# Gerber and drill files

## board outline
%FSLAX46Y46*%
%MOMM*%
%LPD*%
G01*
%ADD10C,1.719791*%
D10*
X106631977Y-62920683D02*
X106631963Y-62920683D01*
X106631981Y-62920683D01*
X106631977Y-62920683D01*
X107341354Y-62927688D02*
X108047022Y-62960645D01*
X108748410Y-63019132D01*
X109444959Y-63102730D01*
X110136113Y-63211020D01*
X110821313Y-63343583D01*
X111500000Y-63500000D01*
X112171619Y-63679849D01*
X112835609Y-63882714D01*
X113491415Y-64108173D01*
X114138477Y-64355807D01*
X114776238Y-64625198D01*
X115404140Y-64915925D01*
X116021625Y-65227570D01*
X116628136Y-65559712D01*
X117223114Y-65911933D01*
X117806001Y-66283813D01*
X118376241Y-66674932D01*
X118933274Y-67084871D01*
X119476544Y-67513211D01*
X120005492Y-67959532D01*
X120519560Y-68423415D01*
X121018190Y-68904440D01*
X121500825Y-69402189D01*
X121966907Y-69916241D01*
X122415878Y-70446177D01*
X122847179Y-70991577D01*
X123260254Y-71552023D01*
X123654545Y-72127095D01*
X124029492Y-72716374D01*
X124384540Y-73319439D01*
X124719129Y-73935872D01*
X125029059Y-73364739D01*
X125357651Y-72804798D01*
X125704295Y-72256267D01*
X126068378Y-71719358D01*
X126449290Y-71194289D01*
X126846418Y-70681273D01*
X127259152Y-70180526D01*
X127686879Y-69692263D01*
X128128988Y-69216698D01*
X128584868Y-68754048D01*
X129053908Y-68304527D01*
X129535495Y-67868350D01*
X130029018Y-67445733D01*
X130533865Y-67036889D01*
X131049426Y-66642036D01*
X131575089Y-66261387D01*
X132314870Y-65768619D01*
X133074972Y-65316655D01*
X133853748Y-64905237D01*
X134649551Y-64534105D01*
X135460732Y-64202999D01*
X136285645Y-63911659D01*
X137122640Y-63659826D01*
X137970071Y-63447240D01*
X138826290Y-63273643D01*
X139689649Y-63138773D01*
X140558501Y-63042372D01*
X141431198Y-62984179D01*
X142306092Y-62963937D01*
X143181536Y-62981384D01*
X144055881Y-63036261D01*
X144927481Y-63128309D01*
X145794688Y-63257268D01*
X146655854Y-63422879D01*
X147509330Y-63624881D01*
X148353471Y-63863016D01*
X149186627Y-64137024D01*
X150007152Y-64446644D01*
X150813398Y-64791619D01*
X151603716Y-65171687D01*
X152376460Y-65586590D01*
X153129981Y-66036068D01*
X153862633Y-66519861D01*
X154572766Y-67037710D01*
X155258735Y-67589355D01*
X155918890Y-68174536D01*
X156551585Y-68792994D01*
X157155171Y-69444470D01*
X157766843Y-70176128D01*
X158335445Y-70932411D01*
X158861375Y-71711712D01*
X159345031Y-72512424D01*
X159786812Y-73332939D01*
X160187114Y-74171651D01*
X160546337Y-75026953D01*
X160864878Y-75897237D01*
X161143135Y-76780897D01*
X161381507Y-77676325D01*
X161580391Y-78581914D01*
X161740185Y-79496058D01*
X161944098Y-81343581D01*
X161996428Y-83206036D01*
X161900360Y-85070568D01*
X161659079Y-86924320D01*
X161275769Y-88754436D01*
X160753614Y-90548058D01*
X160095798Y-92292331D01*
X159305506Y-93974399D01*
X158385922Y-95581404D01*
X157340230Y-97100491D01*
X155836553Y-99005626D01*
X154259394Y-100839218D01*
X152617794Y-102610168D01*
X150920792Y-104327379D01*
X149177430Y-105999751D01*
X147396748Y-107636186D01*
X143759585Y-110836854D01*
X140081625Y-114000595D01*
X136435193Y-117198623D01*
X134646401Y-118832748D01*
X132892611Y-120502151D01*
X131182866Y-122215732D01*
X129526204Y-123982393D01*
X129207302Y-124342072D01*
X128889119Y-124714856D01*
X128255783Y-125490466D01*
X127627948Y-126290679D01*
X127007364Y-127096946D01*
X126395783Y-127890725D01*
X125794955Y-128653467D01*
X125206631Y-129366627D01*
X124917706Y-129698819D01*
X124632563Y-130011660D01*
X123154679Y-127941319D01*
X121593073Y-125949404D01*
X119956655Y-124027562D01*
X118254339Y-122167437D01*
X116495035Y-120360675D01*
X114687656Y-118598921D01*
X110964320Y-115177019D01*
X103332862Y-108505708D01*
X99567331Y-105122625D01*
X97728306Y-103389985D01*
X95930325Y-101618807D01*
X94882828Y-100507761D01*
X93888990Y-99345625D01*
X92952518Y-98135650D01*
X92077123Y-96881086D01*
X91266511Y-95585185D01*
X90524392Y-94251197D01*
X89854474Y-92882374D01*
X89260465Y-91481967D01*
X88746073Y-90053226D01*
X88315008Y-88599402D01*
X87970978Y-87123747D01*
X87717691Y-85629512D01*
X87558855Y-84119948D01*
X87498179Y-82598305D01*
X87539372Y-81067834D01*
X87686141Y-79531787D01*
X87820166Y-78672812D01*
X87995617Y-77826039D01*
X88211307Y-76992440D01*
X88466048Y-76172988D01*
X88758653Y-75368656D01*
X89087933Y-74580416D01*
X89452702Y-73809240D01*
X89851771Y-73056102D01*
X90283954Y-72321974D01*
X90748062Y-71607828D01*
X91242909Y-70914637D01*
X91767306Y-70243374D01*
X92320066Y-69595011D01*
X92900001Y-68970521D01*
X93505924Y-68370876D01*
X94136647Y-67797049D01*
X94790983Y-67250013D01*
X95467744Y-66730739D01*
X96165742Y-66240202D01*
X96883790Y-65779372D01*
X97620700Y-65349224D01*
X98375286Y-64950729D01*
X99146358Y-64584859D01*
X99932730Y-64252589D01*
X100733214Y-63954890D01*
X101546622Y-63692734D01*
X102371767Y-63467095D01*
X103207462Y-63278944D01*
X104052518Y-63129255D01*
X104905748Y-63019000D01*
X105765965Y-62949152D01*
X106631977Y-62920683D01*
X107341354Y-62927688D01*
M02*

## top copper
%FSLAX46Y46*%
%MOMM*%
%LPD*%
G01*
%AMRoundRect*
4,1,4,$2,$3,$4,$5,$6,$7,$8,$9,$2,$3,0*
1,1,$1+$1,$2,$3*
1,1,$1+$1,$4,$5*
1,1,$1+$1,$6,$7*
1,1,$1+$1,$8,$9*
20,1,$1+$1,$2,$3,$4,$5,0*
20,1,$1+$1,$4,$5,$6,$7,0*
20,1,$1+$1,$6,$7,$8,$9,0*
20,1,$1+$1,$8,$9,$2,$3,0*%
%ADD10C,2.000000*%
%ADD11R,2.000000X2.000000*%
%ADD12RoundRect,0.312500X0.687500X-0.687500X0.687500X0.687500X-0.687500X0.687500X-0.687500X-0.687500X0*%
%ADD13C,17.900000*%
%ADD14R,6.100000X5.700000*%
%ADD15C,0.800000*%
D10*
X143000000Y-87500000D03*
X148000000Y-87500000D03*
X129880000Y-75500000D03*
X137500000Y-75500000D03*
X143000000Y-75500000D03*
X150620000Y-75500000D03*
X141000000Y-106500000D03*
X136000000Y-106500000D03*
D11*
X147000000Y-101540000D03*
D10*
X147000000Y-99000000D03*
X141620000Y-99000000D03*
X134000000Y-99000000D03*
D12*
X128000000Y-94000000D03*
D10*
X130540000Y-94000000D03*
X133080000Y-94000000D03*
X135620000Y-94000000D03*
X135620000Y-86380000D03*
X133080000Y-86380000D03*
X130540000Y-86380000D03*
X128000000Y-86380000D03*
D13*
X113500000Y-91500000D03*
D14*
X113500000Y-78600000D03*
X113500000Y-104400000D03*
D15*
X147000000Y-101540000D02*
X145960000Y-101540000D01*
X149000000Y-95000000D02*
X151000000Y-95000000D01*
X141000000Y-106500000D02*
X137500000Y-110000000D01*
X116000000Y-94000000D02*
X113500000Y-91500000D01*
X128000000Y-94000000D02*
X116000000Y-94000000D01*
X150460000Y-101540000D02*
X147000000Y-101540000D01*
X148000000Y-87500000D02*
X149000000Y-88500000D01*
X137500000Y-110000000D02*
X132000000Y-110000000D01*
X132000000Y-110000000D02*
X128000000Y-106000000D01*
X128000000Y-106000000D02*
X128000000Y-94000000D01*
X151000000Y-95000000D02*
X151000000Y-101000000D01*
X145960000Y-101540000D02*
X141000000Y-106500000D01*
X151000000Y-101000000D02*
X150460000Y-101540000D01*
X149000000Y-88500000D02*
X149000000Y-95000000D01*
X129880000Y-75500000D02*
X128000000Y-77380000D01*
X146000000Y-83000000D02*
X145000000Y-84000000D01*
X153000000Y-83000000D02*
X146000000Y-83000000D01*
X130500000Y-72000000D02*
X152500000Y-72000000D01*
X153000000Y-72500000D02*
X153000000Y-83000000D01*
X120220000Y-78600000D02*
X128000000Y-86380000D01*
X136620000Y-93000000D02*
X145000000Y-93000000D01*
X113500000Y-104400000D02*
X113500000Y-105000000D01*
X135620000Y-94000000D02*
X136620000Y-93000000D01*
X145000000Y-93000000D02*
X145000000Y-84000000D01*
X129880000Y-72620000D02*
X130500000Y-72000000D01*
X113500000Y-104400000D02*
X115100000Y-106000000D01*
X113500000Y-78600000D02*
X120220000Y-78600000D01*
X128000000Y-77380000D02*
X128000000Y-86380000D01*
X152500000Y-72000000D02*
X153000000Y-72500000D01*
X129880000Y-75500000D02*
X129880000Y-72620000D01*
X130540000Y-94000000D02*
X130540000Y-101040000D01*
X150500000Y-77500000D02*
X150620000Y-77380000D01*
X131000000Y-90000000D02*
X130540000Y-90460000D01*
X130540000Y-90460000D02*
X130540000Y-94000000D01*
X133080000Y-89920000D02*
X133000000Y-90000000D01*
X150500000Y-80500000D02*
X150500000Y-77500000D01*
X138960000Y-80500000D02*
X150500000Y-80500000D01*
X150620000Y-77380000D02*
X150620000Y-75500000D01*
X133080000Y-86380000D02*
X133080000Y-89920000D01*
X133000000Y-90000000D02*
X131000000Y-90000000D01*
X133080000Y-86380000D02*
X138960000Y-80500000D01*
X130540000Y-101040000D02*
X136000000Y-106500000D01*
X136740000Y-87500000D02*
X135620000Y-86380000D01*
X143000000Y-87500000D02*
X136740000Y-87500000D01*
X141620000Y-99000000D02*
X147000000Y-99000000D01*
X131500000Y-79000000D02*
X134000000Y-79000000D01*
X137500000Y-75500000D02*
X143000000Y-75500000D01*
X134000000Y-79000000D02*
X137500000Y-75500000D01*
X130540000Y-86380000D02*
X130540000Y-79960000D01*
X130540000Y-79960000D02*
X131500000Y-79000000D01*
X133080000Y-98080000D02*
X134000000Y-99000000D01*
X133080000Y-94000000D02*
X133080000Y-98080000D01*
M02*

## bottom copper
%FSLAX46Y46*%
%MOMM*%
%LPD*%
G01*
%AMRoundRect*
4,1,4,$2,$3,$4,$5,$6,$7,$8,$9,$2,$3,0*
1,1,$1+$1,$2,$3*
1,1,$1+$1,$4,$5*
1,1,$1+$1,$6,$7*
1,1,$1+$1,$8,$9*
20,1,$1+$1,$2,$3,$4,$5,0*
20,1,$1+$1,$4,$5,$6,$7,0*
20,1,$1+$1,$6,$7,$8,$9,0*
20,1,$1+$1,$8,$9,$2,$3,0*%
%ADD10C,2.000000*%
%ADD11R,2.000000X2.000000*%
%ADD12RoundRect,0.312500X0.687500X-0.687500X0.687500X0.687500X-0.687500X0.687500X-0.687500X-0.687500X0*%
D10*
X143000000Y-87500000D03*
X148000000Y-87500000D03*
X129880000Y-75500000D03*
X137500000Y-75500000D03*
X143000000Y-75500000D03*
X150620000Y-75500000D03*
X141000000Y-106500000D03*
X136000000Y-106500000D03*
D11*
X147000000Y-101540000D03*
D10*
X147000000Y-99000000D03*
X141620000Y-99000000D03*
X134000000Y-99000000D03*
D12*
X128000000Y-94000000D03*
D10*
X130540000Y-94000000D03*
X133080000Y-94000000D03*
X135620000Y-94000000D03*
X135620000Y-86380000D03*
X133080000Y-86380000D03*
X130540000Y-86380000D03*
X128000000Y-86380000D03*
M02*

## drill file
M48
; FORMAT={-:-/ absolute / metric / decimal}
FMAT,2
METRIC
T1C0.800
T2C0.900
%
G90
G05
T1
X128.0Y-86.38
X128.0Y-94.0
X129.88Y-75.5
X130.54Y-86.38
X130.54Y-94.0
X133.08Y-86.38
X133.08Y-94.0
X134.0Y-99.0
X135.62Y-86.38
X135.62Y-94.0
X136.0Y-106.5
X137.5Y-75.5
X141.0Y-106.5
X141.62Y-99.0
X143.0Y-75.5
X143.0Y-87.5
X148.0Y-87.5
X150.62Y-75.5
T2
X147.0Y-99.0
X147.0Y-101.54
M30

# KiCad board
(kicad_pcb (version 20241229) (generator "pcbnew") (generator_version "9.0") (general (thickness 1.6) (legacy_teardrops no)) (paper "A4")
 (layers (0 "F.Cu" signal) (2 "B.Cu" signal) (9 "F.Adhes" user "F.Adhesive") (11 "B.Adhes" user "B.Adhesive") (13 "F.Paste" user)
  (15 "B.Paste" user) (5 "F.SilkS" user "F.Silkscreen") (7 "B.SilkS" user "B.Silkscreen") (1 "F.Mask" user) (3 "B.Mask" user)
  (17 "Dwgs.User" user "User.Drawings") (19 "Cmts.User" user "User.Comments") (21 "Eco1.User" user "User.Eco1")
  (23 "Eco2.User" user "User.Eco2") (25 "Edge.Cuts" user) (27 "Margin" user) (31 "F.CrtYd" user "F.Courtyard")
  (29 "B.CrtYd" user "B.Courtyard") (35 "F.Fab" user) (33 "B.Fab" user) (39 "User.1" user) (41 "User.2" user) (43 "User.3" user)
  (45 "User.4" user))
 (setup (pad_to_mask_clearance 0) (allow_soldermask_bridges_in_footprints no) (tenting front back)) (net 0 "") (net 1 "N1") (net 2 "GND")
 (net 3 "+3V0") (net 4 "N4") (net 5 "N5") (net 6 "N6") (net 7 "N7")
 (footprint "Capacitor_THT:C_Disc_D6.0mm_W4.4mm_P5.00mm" (layer "F.Cu") (at 143 87.5)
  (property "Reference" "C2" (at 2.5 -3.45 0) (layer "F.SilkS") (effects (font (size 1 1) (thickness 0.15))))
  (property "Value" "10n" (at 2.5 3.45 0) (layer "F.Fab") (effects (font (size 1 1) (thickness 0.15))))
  (pad "1" thru_hole circle (at 0 0) (size 2 2) (drill 0.8) (layers "*.Cu" "*.Mask") (remove_unused_layers no) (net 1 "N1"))
  (pad "2" thru_hole circle (at 5 0) (size 2 2) (drill 0.8) (layers "*.Cu" "*.Mask") (remove_unused_layers no) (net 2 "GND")))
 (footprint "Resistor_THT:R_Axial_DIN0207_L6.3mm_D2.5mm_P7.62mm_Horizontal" (layer "F.Cu") (at 129.88 75.5)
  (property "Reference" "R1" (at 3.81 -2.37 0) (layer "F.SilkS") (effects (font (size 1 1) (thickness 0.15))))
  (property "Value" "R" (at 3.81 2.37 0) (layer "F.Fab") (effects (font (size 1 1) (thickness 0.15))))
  (pad "1" thru_hole circle (at 0 0) (size 2 2) (drill 0.8) (layers "*.Cu" "*.Mask") (remove_unused_layers no) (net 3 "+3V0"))
  (pad "2" thru_hole circle (at 7.62 0) (size 2 2) (drill 0.8) (layers "*.Cu" "*.Mask") (remove_unused_layers no) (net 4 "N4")))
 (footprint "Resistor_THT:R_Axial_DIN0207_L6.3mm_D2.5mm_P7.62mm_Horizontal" (layer "F.Cu") (at 143 75.5)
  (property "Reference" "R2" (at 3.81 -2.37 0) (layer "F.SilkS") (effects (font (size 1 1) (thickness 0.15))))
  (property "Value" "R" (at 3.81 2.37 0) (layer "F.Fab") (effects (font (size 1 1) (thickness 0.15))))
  (pad "1" thru_hole circle (at 0 0) (size 2 2) (drill 0.8) (layers "*.Cu" "*.Mask") (remove_unused_layers no) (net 4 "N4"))
  (pad "2" thru_hole circle (at 7.62 0) (size 2 2) (drill 0.8) (layers "*.Cu" "*.Mask") (remove_unused_layers no) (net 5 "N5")))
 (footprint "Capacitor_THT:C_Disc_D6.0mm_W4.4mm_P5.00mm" (layer "F.Cu") (at 141 106.5 180)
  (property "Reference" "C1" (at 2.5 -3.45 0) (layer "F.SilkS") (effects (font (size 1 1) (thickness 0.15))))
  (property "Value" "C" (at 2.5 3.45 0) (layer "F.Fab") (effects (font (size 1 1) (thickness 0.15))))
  (pad "1" thru_hole circle (at 0 0 180) (size 2 2) (drill 0.8) (layers "*.Cu" "*.Mask") (remove_unused_layers no) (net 2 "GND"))
  (pad "2" thru_hole circle (at 5 0 180) (size 2 2) (drill 0.8) (layers "*.Cu" "*.Mask") (remove_unused_layers no) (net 5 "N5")))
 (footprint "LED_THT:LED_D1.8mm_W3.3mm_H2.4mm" (layer "F.Cu") (at 147 101.54 90)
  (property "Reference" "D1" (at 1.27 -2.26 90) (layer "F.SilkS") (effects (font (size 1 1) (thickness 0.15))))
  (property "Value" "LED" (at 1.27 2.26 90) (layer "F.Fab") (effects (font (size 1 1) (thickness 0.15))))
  (pad "1" thru_hole rect (at 0 0 90) (size 2 2) (drill 0.9) (layers "*.Cu" "*.Mask") (remove_unused_layers no) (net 2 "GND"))
  (pad "2" thru_hole circle (at 2.54 0 90) (size 2 2) (drill 0.9) (layers "*.Cu" "*.Mask") (remove_unused_layers no) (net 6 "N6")))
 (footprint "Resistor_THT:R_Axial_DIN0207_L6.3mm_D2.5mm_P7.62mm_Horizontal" (layer "F.Cu") (at 141.62 99 180)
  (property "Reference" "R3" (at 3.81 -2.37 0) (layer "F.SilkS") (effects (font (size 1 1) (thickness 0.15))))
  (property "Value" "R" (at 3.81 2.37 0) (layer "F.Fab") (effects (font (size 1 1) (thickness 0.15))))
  (pad "1" thru_hole circle (at 0 0 180) (size 2 2) (drill 0.8) (layers "*.Cu" "*.Mask") (remove_unused_layers no) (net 6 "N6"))
  (pad "2" thru_hole circle (at 7.62 0 180) (size 2 2) (drill 0.8) (layers "*.Cu" "*.Mask") (remove_unused_layers no) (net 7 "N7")))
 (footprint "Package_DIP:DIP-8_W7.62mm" (layer "F.Cu") (at 128 94 90)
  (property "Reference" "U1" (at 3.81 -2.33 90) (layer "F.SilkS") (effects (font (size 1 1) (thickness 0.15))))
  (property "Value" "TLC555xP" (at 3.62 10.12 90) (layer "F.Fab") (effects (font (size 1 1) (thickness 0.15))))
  (pad "1" thru_hole roundrect (at 0 0 90) (size 2 2) (drill 0.8) (layers "*.Cu" "*.Mask") (remove_unused_layers no)
   (roundrect_rratio 0.15625) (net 2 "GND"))
  (pad "2" thru_hole circle (at 0 2.54 90) (size 2 2) (drill 0.8) (layers "*.Cu" "*.Mask") (remove_unused_layers no) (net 5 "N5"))
  (pad "3" thru_hole circle (at 0 5.08 90) (size 2 2) (drill 0.8) (layers "*.Cu" "*.Mask") (remove_unused_layers no) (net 7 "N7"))
  (pad "4" thru_hole circle (at 0 7.62 90) (size 2 2) (drill 0.8) (layers "*.Cu" "*.Mask") (remove_unused_layers no) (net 3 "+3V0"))
  (pad "5" thru_hole circle (at 7.62 7.62 90) (size 2 2) (drill 0.8) (layers "*.Cu" "*.Mask") (remove_unused_layers no) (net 1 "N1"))
  (pad "6" thru_hole circle (at 7.62 5.08 90) (size 2 2) (drill 0.8) (layers "*.Cu" "*.Mask") (remove_unused_layers no) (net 5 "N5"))
  (pad "7" thru_hole circle (at 7.62 2.54 90) (size 2 2) (drill 0.8) (layers "*.Cu" "*.Mask") (remove_unused_layers no) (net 4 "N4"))
  (pad "8" thru_hole circle (at 7.62 0 90) (size 2 2) (drill 0.8) (layers "*.Cu" "*.Mask") (remove_unused_layers no) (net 3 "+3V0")))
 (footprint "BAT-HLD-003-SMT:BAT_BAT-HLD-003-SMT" (layer "F.Cu") (at 113.5 91.5 -90)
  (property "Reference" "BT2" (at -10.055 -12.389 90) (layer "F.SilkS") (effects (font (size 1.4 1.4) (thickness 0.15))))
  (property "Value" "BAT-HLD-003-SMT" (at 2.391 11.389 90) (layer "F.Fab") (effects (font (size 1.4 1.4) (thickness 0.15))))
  (pad "N" smd circle (at 0 0 270) (size 17.9 17.9) (layers "F.Cu" "F.Mask") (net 2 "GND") (solder_mask_margin 0.102))
  (pad "P1" smd rect (at -12.9 0 270) (size 5.7 6.1) (layers "F.Cu" "F.Mask" "F.Paste") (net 3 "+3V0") (solder_mask_margin 0.102))
  (pad "P2" smd rect (at 12.9 0 270) (size 5.7 6.1) (layers "F.Cu" "F.Mask" "F.Paste") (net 3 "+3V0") (solder_mask_margin 0.102)))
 (gr_poly
  (pts (xy 106.631977 62.920683) (xy 106.631963 62.920683) (xy 106.631981 62.920683)) (stroke (width 1.719791) (type solid)) (fill no)
  (layer "Edge.Cuts"))
 (gr_poly
  (pts (xy 107.341354 62.927688) (xy 108.047022 62.960645) (xy 108.74841 63.019132) (xy 109.444959 63.10273) (xy 110.136113 63.21102)
   (xy 110.821313 63.343583) (xy 111.5 63.5) (xy 112.171619 63.679849) (xy 112.835609 63.882714) (xy 113.491415 64.108173)
   (xy 114.138477 64.355807) (xy 114.776238 64.625198) (xy 115.40414 64.915925) (xy 116.021625 65.22757) (xy 116.628136 65.559712)
   (xy 117.223114 65.911933) (xy 117.806001 66.283813) (xy 118.376241 66.674932) (xy 118.933274 67.084871) (xy 119.476544 67.513211)
   (xy 120.005492 67.959532) (xy 120.51956 68.423415) (xy 121.01819 68.90444) (xy 121.500825 69.402189) (xy 121.966907 69.916241)
   (xy 122.415878 70.446177) (xy 122.847179 70.991577) (xy 123.260254 71.552023) (xy 123.654545 72.127095) (xy 124.029492 72.716374)
   (xy 124.38454 73.319439) (xy 124.719129 73.935872) (xy 125.029059 73.364739) (xy 125.357651 72.804798) (xy 125.704295 72.256267)
   (xy 126.068378 71.719358) (xy 126.44929 71.194289) (xy 126.846418 70.681273) (xy 127.259152 70.180526) (xy 127.686879 69.692263)
   (xy 128.128988 69.216698) (xy 128.584868 68.754048) (xy 129.053908 68.304527) (xy 129.535495 67.86835) (xy 130.029018 67.445733)
   (xy 130.533865 67.036889) (xy 131.049426 66.642036) (xy 131.575089 66.261387) (xy 132.31487 65.768619) (xy 133.074972 65.316655)
   (xy 133.853748 64.905237) (xy 134.649551 64.534105) (xy 135.460732 64.202999) (xy 136.285645 63.911659) (xy 137.12264 63.659826)
   (xy 137.970071 63.44724) (xy 138.82629 63.273643) (xy 139.689649 63.138773) (xy 140.558501 63.042372) (xy 141.431198 62.984179)
   (xy 142.306092 62.963937) (xy 143.181536 62.981384) (xy 144.055881 63.036261) (xy 144.927481 63.128309) (xy 145.794688 63.257268)
   (xy 146.655854 63.422879) (xy 147.50933 63.624881) (xy 148.353471 63.863016) (xy 149.186627 64.137024) (xy 150.007152 64.446644)
   (xy 150.813398 64.791619) (xy 151.603716 65.171687) (xy 152.37646 65.58659) (xy 153.129981 66.036068) (xy 153.862633 66.519861)
   (xy 154.572766 67.03771) (xy 155.258735 67.589355) (xy 155.91889 68.174536) (xy 156.551585 68.792994) (xy 157.155171 69.44447)
   (xy 157.766843 70.176128) (xy 158.335445 70.932411) (xy 158.861375 71.711712) (xy 159.345031 72.512424) (xy 159.786812 73.332939)
   (xy 160.187114 74.171651) (xy 160.546337 75.026953) (xy 160.864878 75.897237) (xy 161.143135 76.780897) (xy 161.381507 77.676325)
   (xy 161.580391 78.581914) (xy 161.740185 79.496058) (xy 161.944098 81.343581) (xy 161.996428 83.206036) (xy 161.90036 85.070568)
   (xy 161.659079 86.92432) (xy 161.275769 88.754436) (xy 160.753614 90.548058) (xy 160.095798 92.292331) (xy 159.305506 93.974399)
   (xy 158.385922 95.581404) (xy 157.34023 97.100491) (xy 155.836553 99.005626) (xy 154.259394 100.839218) (xy 152.617794 102.610168)
   (xy 150.920792 104.327379) (xy 149.17743 105.999751) (xy 147.396748 107.636186) (xy 143.759585 110.836854) (xy 140.081625 114.000595)
   (xy 136.435193 117.198623) (xy 134.646401 118.832748) (xy 132.892611 120.502151) (xy 131.182866 122.215732) (xy 129.526204 123.982393)
   (xy 129.207302 124.342072) (xy 128.889119 124.714856) (xy 128.255783 125.490466) (xy 127.627948 126.290679) (xy 127.007364 127.096946)
   (xy 126.395783 127.890725) (xy 125.794955 128.653467) (xy 125.206631 129.366627) (xy 124.917706 129.698819) (xy 124.632563 130.01166)
   (xy 123.154679 127.941319) (xy 121.593073 125.949404) (xy 119.956655 124.027562) (xy 118.254339 122.167437) (xy 116.495035 120.360675)
   (xy 114.687656 118.598921) (xy 110.96432 115.177019) (xy 103.332862 108.505708) (xy 99.567331 105.122625) (xy 97.728306 103.389985)
   (xy 95.930325 101.618807) (xy 94.882828 100.507761) (xy 93.88899 99.345625) (xy 92.952518 98.13565) (xy 92.077123 96.881086)
   (xy 91.266511 95.585185) (xy 90.524392 94.251197) (xy 89.854474 92.882374) (xy 89.260465 91.481967) (xy 88.746073 90.053226)
   (xy 88.315008 88.599402) (xy 87.970978 87.123747) (xy 87.717691 85.629512) (xy 87.558855 84.119948) (xy 87.498179 82.598305)
   (xy 87.539372 81.067834) (xy 87.686141 79.531787) (xy 87.820166 78.672812) (xy 87.995617 77.826039) (xy 88.211307 76.99244)
   (xy 88.466048 76.172988) (xy 88.758653 75.368656) (xy 89.087933 74.580416) (xy 89.452702 73.80924) (xy 89.851771 73.056102)
   (xy 90.283954 72.321974) (xy 90.748062 71.607828) (xy 91.242909 70.914637) (xy 91.767306 70.243374) (xy 92.320066 69.595011)
   (xy 92.900001 68.970521) (xy 93.505924 68.370876) (xy 94.136647 67.797049) (xy 94.790983 67.250013) (xy 95.467744 66.730739)
   (xy 96.165742 66.240202) (xy 96.88379 65.779372) (xy 97.6207 65.349224) (xy 98.375286 64.950729) (xy 99.146358 64.584859)
   (xy 99.93273 64.252589) (xy 100.733214 63.95489) (xy 101.546622 63.692734) (xy 102.371767 63.467095) (xy 103.207462 63.278944)
   (xy 104.052518 63.129255) (xy 104.905748 63.019) (xy 105.765965 62.949152) (xy 106.631977 62.920683))
  (stroke (width 1.719791) (type solid)) (fill no) (layer "Edge.Cuts"))
 (segment (start 147 101.54) (end 145.96 101.54) (width 0.8) (layer "F.Cu") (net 2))
 (segment (start 149 95) (end 151 95) (width 0.8) (layer "F.Cu") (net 2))
 (segment (start 141 106.5) (end 137.5 110) (width 0.8) (layer "F.Cu") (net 2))
 (segment (start 116 94) (end 113.5 91.5) (width 0.8) (layer "F.Cu") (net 2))
 (segment (start 128 94) (end 116 94) (width 0.8) (layer "F.Cu") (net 2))
 (segment (start 150.46 101.54) (end 147 101.54) (width 0.8) (layer "F.Cu") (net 2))
 (segment (start 148 87.5) (end 149 88.5) (width 0.8) (layer "F.Cu") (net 2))
 (segment (start 137.5 110) (end 132 110) (width 0.8) (layer "F.Cu") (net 2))
 (segment (start 132 110) (end 128 106) (width 0.8) (layer "F.Cu") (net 2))
 (segment (start 128 106) (end 128 94) (width 0.8) (layer "F.Cu") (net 2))
 (segment (start 151 95) (end 151 101) (width 0.8) (layer "F.Cu") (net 2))
 (segment (start 145.96 101.54) (end 141 106.5) (width 0.8) (layer "F.Cu") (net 2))
 (segment (start 151 101) (end 150.46 101.54) (width 0.8) (layer "F.Cu") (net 2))
 (segment (start 149 88.5) (end 149 95) (width 0.8) (layer "F.Cu") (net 2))
 (segment (start 129.88 75.5) (end 128 77.38) (width 0.8) (layer "F.Cu") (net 3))
 (segment (start 146 83) (end 145 84) (width 0.8) (layer "F.Cu") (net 3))
 (segment (start 153 83) (end 146 83) (width 0.8) (layer "F.Cu") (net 3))
 (segment (start 130.5 72) (end 152.5 72) (width 0.8) (layer "F.Cu") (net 3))
 (segment (start 153 72.5) (end 153 83) (width 0.8) (layer "F.Cu") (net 3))
 (segment (start 120.22 78.6) (end 128 86.38) (width 0.8) (layer "F.Cu") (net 3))
 (segment (start 136.62 93) (end 145 93) (width 0.8) (layer "F.Cu") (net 3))
 (segment (start 113.5 104.4) (end 113.5 105) (width 0.8) (layer "F.Cu") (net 3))
 (segment (start 135.62 94) (end 136.62 93) (width 0.8) (layer "F.Cu") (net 3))
 (segment (start 145 93) (end 145 84) (width 0.8) (layer "F.Cu") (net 3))
 (segment (start 129.88 72.62) (end 130.5 72) (width 0.8) (layer "F.Cu") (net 3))
 (segment (start 113.5 104.4) (end 115.1 106) (width 0.8) (layer "F.Cu") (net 3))
 (segment (start 113.5 78.6) (end 120.22 78.6) (width 0.8) (layer "F.Cu") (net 3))
 (segment (start 128 77.38) (end 128 86.38) (width 0.8) (layer "F.Cu") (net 3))
 (segment (start 152.5 72) (end 153 72.5) (width 0.8) (layer "F.Cu") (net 3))
 (segment (start 129.88 75.5) (end 129.88 72.62) (width 0.8) (layer "F.Cu") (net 3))
 (segment (start 130.54 94) (end 130.54 101.04) (width 0.8) (layer "F.Cu") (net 5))
 (segment (start 150.5 77.5) (end 150.62 77.38) (width 0.8) (layer "F.Cu") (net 5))
 (segment (start 131 90) (end 130.54 90.46) (width 0.8) (layer "F.Cu") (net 5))
 (segment (start 130.54 90.46) (end 130.54 94) (width 0.8) (layer "F.Cu") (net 5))
 (segment (start 133.08 89.92) (end 133 90) (width 0.8) (layer "F.Cu") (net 5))
 (segment (start 150.5 80.5) (end 150.5 77.5) (width 0.8) (layer "F.Cu") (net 5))
 (segment (start 138.96 80.5) (end 150.5 80.5) (width 0.8) (layer "F.Cu") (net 5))
 (segment (start 150.62 77.38) (end 150.62 75.5) (width 0.8) (layer "F.Cu") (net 5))
 (segment (start 133.08 86.38) (end 133.08 89.92) (width 0.8) (layer "F.Cu") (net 5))
 (segment (start 133 90) (end 131 90) (width 0.8) (layer "F.Cu") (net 5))
 (segment (start 133.08 86.38) (end 138.96 80.5) (width 0.8) (layer "F.Cu") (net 5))
 (segment (start 130.54 101.04) (end 136 106.5) (width 0.8) (layer "F.Cu") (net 5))
 (segment (start 136.74 87.5) (end 135.62 86.38) (width 0.8) (layer "F.Cu") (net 1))
 (segment (start 143 87.5) (end 136.74 87.5) (width 0.8) (layer "F.Cu") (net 1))
 (segment (start 141.62 99) (end 147 99) (width 0.8) (layer "F.Cu") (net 6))
 (segment (start 131.5 79) (end 134 79) (width 0.8) (layer "F.Cu") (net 4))
 (segment (start 137.5 75.5) (end 143 75.5) (width 0.8) (layer "F.Cu") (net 4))
 (segment (start 134 79) (end 137.5 75.5) (width 0.8) (layer "F.Cu") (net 4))
 (segment (start 130.54 86.38) (end 130.54 79.96) (width 0.8) (layer "F.Cu") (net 4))
 (segment (start 130.54 79.96) (end 131.5 79) (width 0.8) (layer "F.Cu") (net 4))
 (segment (start 133.08 98.08) (end 134 99) (width 0.8) (layer "F.Cu") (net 7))
 (segment (start 133.08 94) (end 133.08 98.08) (width 0.8) (layer "F.Cu") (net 7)))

